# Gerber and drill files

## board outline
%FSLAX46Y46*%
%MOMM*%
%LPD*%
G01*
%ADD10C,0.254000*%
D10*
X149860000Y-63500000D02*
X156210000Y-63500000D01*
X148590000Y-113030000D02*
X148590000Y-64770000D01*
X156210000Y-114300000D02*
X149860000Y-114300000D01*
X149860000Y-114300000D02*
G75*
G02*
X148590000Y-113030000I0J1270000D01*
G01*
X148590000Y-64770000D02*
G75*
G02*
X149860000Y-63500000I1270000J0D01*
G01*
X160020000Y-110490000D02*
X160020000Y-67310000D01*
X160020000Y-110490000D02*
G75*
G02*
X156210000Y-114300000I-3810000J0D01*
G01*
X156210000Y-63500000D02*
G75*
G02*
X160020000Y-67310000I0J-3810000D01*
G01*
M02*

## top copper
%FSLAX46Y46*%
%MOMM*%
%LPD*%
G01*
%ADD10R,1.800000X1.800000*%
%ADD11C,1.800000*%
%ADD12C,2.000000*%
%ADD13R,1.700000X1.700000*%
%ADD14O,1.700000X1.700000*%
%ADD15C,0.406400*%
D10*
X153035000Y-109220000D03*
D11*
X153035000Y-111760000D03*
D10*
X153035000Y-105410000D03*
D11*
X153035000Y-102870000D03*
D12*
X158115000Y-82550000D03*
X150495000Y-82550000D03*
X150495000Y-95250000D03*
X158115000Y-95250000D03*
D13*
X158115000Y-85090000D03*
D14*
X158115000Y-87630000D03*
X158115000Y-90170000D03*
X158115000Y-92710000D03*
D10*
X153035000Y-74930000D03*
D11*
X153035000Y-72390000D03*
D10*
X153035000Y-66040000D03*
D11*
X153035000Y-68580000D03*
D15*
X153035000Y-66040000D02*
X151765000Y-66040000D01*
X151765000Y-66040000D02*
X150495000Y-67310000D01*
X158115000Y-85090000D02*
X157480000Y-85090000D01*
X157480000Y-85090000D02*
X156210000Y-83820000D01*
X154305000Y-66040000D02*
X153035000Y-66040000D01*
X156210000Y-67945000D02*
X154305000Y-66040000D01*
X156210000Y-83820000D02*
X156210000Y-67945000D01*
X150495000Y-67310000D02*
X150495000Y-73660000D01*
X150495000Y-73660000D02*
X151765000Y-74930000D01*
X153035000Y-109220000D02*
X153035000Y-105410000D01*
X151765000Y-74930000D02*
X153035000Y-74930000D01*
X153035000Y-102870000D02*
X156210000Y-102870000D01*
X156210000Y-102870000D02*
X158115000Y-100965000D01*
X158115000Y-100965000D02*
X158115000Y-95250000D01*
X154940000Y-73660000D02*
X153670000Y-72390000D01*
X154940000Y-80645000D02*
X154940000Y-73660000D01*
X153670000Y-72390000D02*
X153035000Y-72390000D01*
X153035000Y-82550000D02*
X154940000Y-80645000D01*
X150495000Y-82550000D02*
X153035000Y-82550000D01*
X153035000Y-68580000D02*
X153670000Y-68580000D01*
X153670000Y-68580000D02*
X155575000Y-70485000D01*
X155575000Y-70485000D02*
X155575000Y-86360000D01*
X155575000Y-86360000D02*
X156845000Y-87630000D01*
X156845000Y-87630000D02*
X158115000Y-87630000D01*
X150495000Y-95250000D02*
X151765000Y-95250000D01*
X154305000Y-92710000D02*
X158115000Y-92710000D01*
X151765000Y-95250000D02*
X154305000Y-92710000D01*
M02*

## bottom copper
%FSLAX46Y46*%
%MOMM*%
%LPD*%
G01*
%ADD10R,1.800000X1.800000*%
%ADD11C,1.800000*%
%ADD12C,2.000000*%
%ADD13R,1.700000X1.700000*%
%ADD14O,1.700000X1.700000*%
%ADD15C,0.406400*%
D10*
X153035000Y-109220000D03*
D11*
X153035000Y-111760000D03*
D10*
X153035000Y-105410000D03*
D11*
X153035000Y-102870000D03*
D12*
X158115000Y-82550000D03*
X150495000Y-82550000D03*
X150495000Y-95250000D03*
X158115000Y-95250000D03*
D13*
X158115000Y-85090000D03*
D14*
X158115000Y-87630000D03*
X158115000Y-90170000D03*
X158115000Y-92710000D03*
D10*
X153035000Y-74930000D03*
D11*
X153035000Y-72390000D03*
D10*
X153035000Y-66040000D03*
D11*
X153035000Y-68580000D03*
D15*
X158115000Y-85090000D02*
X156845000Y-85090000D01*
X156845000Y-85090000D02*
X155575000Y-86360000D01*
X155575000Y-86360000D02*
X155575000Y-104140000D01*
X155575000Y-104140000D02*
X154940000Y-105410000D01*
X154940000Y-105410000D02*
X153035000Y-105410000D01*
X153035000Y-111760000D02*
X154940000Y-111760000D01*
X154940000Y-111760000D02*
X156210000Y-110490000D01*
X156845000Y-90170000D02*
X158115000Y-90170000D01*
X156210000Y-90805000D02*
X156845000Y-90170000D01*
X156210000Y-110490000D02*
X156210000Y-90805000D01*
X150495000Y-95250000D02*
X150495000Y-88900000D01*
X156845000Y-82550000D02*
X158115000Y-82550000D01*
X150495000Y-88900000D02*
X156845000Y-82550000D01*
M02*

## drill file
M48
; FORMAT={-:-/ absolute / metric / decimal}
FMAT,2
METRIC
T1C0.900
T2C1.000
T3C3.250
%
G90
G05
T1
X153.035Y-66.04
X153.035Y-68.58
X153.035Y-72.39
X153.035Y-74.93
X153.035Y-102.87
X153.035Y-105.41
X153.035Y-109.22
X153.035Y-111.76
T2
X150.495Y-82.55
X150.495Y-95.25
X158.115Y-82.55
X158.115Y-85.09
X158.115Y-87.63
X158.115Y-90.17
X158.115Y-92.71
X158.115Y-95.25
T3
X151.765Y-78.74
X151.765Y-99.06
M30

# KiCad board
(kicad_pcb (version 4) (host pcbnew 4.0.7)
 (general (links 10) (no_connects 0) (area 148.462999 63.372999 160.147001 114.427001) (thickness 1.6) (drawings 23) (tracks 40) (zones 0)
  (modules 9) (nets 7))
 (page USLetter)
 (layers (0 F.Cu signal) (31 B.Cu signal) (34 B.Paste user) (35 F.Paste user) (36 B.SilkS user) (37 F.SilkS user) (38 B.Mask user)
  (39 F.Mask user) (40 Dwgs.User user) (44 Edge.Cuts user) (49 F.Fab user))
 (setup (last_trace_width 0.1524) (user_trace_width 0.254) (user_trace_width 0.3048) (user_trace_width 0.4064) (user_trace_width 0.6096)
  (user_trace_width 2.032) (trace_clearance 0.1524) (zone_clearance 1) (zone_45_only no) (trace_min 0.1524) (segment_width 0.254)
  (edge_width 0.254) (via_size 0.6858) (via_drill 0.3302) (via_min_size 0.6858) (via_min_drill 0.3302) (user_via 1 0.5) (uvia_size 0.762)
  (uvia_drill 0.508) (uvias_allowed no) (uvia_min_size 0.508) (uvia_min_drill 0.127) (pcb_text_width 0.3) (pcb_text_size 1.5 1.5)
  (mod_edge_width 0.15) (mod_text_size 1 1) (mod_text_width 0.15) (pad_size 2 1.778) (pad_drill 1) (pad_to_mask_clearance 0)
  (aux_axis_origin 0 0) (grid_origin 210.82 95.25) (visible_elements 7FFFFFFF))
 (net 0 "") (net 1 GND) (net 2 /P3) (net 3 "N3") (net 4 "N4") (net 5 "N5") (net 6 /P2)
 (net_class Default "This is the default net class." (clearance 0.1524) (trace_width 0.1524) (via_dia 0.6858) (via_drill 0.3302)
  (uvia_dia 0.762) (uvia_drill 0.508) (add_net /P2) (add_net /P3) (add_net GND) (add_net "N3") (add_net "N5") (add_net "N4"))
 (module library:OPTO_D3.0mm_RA (layer F.Cu) (at 153.035 111.76 90)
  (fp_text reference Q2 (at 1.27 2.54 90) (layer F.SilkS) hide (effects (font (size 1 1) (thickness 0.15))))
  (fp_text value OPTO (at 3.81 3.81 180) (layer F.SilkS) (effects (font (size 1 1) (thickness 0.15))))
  (pad 1 thru_hole rect (at 2.54 0 90) (size 1.8 1.8) (drill 0.9) (layers *.Cu *.Mask) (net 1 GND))
  (pad 3 thru_hole circle (at 0 0 90) (size 1.8 1.8) (drill 0.9) (layers *.Cu *.Mask) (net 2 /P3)))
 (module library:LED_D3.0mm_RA (layer F.Cu) (at 153.035 105.41 90)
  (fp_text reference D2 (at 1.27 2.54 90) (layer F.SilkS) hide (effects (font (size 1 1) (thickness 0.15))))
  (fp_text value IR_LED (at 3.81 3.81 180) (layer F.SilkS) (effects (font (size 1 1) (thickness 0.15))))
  (pad 1 thru_hole rect (at 0 0 90) (size 1.8 1.8) (drill 0.9) (layers *.Cu *.Mask) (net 1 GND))
  (pad 2 thru_hole circle (at 2.54 0 90) (size 1.8 1.8) (drill 0.9) (layers *.Cu *.Mask) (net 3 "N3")))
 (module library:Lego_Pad (layer F.Cu) (at 151.765 99.06)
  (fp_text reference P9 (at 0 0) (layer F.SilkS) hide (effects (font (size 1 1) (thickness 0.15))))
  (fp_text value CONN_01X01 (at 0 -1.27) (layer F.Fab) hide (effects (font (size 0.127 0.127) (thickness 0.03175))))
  (pad "" np_thru_hole circle (at 0 0) (size 3.25 3.25) (drill 3.25) (layers *.Cu *.Mask)))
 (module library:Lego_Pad (layer F.Cu) (at 151.765 78.74)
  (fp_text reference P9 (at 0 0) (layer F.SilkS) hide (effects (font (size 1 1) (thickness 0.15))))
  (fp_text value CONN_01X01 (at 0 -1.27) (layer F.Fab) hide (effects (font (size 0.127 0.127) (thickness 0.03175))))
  (pad "" np_thru_hole circle (at 0 0) (size 3.25 3.25) (drill 3.25) (layers *.Cu *.Mask)))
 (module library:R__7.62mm (layer F.Cu) (at 154.305 82.55 180)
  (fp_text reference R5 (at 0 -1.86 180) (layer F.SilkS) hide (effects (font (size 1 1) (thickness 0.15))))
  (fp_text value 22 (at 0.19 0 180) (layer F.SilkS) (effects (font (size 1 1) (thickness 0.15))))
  (pad 1 thru_hole circle (at -3.81 0 180) (size 2 2) (drill 1) (layers *.Cu *.Mask) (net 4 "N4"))
  (pad 2 thru_hole circle (at 3.81 0 180) (size 2 2) (drill 1) (layers *.Cu *.Mask) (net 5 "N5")))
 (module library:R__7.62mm (layer F.Cu) (at 154.305 95.25)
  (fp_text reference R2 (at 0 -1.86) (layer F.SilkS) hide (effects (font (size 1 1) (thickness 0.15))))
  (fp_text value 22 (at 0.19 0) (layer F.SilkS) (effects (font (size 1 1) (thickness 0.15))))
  (pad 1 thru_hole circle (at -3.81 0) (size 2 2) (drill 1) (layers *.Cu *.Mask) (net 4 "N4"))
  (pad 2 thru_hole circle (at 3.81 0) (size 2 2) (drill 1) (layers *.Cu *.Mask) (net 3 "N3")))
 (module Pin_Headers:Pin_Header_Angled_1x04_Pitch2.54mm (layer B.Cu) (at 158.115 85.09 180)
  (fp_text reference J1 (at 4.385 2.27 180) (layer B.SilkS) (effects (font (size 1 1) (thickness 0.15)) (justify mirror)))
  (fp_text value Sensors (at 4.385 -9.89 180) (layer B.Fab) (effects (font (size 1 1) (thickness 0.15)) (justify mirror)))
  (pad 1 thru_hole rect (at 0 0 180) (size 1.7 1.7) (drill 1) (layers *.Cu *.Mask) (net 1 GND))
  (pad 2 thru_hole oval (at 0 -2.54 180) (size 1.7 1.7) (drill 1) (layers *.Cu *.Mask) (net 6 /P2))
  (pad 3 thru_hole oval (at 0 -5.08 180) (size 1.7 1.7) (drill 1) (layers *.Cu *.Mask) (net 2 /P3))
  (pad 4 thru_hole oval (at 0 -7.62 180) (size 1.7 1.7) (drill 1) (layers *.Cu *.Mask) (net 4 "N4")))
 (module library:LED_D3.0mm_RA (layer F.Cu) (at 153.035 74.93 90)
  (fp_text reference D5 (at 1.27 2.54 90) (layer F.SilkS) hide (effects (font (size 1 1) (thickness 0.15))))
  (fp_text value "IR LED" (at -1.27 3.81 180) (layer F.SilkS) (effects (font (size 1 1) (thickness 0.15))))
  (pad 1 thru_hole rect (at 0 0 90) (size 1.8 1.8) (drill 0.9) (layers *.Cu *.Mask) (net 1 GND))
  (pad 2 thru_hole circle (at 2.54 0 90) (size 1.8 1.8) (drill 0.9) (layers *.Cu *.Mask) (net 5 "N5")))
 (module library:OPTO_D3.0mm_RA (layer F.Cu) (at 153.035 68.58 90)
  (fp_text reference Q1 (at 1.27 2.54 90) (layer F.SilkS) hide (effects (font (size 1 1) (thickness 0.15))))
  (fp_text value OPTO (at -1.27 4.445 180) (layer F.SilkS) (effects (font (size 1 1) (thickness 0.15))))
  (pad 1 thru_hole rect (at 2.54 0 90) (size 1.8 1.8) (drill 0.9) (layers *.Cu *.Mask) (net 1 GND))
  (pad 3 thru_hole circle (at 0 0 90) (size 1.8 1.8) (drill 0.9) (layers *.Cu *.Mask) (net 6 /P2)))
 (gr_line (start 149.86 63.5) (end 156.21 63.5) (angle 90) (layer Edge.Cuts) (width 0.254))
 (gr_line (start 148.59 113.03) (end 148.59 64.77) (angle 90) (layer Edge.Cuts) (width 0.254))
 (gr_line (start 156.21 114.3) (end 149.86 114.3) (angle 90) (layer Edge.Cuts) (width 0.254))
 (gr_arc (start 149.86 113.03) (end 149.86 114.3) (angle 90) (layer Edge.Cuts) (width 0.254))
 (gr_arc (start 149.86 64.77) (end 148.59 64.77) (angle 90) (layer Edge.Cuts) (width 0.254))
 (gr_line (start 160.02 110.49) (end 160.02 67.31) (angle 90) (layer Edge.Cuts) (width 0.254))
 (gr_arc (start 156.21 110.49) (end 160.02 110.49) (angle 90) (layer Edge.Cuts) (width 0.254))
 (gr_arc (start 156.21 67.31) (end 156.21 63.5) (angle 90) (layer Edge.Cuts) (width 0.254))
 (segment (start 153.035 66.04) (end 151.765 66.04) (width 0.4064) (layer F.Cu) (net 1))
 (segment (start 151.765 66.04) (end 150.495 67.31) (width 0.4064) (layer F.Cu) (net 1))
 (segment (start 158.115 85.09) (end 157.48 85.09) (width 0.4064) (layer F.Cu) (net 1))
 (segment (start 157.48 85.09) (end 156.21 83.82) (width 0.4064) (layer F.Cu) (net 1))
 (segment (start 154.305 66.04) (end 153.035 66.04) (width 0.4064) (layer F.Cu) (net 1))
 (segment (start 156.21 67.945) (end 154.305 66.04) (width 0.4064) (layer F.Cu) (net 1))
 (segment (start 156.21 83.82) (end 156.21 67.945) (width 0.4064) (layer F.Cu) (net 1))
 (segment (start 158.115 85.09) (end 156.845 85.09) (width 0.4064) (layer B.Cu) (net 1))
 (segment (start 156.845 85.09) (end 155.575 86.36) (width 0.4064) (layer B.Cu) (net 1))
 (segment (start 155.575 86.36) (end 155.575 104.14) (width 0.4064) (layer B.Cu) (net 1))
 (segment (start 155.575 104.14) (end 154.94 105.41) (width 0.4064) (layer B.Cu) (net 1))
 (segment (start 150.495 67.31) (end 150.495 73.66) (width 0.4064) (layer F.Cu) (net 1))
 (segment (start 150.495 73.66) (end 151.765 74.93) (width 0.4064) (layer F.Cu) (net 1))
 (segment (start 154.94 105.41) (end 153.035 105.41) (width 0.4064) (layer B.Cu) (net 1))
 (segment (start 153.035 109.22) (end 153.035 105.41) (width 0.4064) (layer F.Cu) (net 1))
 (segment (start 151.765 74.93) (end 153.035 74.93) (width 0.4064) (layer F.Cu) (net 1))
 (segment (start 153.035 102.87) (end 156.21 102.87) (width 0.4064) (layer F.Cu) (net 3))
 (segment (start 156.21 102.87) (end 158.115 100.965) (width 0.4064) (layer F.Cu) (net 3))
 (segment (start 158.115 100.965) (end 158.115 95.25) (width 0.4064) (layer F.Cu) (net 3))
 (segment (start 154.94 73.66) (end 153.67 72.39) (width 0.4064) (layer F.Cu) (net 5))
 (segment (start 154.94 80.645) (end 154.94 73.66) (width 0.4064) (layer F.Cu) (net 5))
 (segment (start 153.67 72.39) (end 153.035 72.39) (width 0.4064) (layer F.Cu) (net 5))
 (segment (start 153.035 82.55) (end 154.94 80.645) (width 0.4064) (layer F.Cu) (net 5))
 (segment (start 150.495 82.55) (end 153.035 82.55) (width 0.4064) (layer F.Cu) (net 5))
 (segment (start 153.035 111.76) (end 154.94 111.76) (width 0.4064) (layer B.Cu) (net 2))
 (segment (start 154.94 111.76) (end 156.21 110.49) (width 0.4064) (layer B.Cu) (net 2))
 (segment (start 156.845 90.17) (end 158.115 90.17) (width 0.4064) (layer B.Cu) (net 2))
 (segment (start 156.21 90.805) (end 156.845 90.17) (width 0.4064) (layer B.Cu) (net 2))
 (segment (start 156.21 110.49) (end 156.21 90.805) (width 0.4064) (layer B.Cu) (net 2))
 (segment (start 153.035 68.58) (end 153.67 68.58) (width 0.4064) (layer F.Cu) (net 6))
 (segment (start 153.67 68.58) (end 155.575 70.485) (width 0.4064) (layer F.Cu) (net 6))
 (segment (start 155.575 70.485) (end 155.575 86.36) (width 0.4064) (layer F.Cu) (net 6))
 (segment (start 155.575 86.36) (end 156.845 87.63) (width 0.4064) (layer F.Cu) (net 6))
 (segment (start 156.845 87.63) (end 158.115 87.63) (width 0.4064) (layer F.Cu) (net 6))
 (segment (start 150.495 95.25) (end 150.495 88.9) (width 0.4064) (layer B.Cu) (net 4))
 (segment (start 156.845 82.55) (end 158.115 82.55) (width 0.4064) (layer B.Cu) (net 4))
 (segment (start 150.495 88.9) (end 156.845 82.55) (width 0.4064) (layer B.Cu) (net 4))
 (segment (start 150.495 95.25) (end 151.765 95.25) (width 0.4064) (layer F.Cu) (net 4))
 (segment (start 154.305 92.71) (end 158.115 92.71) (width 0.4064) (layer F.Cu) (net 4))
 (segment (start 151.765 95.25) (end 154.305 92.71) (width 0.4064) (layer F.Cu) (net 4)))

